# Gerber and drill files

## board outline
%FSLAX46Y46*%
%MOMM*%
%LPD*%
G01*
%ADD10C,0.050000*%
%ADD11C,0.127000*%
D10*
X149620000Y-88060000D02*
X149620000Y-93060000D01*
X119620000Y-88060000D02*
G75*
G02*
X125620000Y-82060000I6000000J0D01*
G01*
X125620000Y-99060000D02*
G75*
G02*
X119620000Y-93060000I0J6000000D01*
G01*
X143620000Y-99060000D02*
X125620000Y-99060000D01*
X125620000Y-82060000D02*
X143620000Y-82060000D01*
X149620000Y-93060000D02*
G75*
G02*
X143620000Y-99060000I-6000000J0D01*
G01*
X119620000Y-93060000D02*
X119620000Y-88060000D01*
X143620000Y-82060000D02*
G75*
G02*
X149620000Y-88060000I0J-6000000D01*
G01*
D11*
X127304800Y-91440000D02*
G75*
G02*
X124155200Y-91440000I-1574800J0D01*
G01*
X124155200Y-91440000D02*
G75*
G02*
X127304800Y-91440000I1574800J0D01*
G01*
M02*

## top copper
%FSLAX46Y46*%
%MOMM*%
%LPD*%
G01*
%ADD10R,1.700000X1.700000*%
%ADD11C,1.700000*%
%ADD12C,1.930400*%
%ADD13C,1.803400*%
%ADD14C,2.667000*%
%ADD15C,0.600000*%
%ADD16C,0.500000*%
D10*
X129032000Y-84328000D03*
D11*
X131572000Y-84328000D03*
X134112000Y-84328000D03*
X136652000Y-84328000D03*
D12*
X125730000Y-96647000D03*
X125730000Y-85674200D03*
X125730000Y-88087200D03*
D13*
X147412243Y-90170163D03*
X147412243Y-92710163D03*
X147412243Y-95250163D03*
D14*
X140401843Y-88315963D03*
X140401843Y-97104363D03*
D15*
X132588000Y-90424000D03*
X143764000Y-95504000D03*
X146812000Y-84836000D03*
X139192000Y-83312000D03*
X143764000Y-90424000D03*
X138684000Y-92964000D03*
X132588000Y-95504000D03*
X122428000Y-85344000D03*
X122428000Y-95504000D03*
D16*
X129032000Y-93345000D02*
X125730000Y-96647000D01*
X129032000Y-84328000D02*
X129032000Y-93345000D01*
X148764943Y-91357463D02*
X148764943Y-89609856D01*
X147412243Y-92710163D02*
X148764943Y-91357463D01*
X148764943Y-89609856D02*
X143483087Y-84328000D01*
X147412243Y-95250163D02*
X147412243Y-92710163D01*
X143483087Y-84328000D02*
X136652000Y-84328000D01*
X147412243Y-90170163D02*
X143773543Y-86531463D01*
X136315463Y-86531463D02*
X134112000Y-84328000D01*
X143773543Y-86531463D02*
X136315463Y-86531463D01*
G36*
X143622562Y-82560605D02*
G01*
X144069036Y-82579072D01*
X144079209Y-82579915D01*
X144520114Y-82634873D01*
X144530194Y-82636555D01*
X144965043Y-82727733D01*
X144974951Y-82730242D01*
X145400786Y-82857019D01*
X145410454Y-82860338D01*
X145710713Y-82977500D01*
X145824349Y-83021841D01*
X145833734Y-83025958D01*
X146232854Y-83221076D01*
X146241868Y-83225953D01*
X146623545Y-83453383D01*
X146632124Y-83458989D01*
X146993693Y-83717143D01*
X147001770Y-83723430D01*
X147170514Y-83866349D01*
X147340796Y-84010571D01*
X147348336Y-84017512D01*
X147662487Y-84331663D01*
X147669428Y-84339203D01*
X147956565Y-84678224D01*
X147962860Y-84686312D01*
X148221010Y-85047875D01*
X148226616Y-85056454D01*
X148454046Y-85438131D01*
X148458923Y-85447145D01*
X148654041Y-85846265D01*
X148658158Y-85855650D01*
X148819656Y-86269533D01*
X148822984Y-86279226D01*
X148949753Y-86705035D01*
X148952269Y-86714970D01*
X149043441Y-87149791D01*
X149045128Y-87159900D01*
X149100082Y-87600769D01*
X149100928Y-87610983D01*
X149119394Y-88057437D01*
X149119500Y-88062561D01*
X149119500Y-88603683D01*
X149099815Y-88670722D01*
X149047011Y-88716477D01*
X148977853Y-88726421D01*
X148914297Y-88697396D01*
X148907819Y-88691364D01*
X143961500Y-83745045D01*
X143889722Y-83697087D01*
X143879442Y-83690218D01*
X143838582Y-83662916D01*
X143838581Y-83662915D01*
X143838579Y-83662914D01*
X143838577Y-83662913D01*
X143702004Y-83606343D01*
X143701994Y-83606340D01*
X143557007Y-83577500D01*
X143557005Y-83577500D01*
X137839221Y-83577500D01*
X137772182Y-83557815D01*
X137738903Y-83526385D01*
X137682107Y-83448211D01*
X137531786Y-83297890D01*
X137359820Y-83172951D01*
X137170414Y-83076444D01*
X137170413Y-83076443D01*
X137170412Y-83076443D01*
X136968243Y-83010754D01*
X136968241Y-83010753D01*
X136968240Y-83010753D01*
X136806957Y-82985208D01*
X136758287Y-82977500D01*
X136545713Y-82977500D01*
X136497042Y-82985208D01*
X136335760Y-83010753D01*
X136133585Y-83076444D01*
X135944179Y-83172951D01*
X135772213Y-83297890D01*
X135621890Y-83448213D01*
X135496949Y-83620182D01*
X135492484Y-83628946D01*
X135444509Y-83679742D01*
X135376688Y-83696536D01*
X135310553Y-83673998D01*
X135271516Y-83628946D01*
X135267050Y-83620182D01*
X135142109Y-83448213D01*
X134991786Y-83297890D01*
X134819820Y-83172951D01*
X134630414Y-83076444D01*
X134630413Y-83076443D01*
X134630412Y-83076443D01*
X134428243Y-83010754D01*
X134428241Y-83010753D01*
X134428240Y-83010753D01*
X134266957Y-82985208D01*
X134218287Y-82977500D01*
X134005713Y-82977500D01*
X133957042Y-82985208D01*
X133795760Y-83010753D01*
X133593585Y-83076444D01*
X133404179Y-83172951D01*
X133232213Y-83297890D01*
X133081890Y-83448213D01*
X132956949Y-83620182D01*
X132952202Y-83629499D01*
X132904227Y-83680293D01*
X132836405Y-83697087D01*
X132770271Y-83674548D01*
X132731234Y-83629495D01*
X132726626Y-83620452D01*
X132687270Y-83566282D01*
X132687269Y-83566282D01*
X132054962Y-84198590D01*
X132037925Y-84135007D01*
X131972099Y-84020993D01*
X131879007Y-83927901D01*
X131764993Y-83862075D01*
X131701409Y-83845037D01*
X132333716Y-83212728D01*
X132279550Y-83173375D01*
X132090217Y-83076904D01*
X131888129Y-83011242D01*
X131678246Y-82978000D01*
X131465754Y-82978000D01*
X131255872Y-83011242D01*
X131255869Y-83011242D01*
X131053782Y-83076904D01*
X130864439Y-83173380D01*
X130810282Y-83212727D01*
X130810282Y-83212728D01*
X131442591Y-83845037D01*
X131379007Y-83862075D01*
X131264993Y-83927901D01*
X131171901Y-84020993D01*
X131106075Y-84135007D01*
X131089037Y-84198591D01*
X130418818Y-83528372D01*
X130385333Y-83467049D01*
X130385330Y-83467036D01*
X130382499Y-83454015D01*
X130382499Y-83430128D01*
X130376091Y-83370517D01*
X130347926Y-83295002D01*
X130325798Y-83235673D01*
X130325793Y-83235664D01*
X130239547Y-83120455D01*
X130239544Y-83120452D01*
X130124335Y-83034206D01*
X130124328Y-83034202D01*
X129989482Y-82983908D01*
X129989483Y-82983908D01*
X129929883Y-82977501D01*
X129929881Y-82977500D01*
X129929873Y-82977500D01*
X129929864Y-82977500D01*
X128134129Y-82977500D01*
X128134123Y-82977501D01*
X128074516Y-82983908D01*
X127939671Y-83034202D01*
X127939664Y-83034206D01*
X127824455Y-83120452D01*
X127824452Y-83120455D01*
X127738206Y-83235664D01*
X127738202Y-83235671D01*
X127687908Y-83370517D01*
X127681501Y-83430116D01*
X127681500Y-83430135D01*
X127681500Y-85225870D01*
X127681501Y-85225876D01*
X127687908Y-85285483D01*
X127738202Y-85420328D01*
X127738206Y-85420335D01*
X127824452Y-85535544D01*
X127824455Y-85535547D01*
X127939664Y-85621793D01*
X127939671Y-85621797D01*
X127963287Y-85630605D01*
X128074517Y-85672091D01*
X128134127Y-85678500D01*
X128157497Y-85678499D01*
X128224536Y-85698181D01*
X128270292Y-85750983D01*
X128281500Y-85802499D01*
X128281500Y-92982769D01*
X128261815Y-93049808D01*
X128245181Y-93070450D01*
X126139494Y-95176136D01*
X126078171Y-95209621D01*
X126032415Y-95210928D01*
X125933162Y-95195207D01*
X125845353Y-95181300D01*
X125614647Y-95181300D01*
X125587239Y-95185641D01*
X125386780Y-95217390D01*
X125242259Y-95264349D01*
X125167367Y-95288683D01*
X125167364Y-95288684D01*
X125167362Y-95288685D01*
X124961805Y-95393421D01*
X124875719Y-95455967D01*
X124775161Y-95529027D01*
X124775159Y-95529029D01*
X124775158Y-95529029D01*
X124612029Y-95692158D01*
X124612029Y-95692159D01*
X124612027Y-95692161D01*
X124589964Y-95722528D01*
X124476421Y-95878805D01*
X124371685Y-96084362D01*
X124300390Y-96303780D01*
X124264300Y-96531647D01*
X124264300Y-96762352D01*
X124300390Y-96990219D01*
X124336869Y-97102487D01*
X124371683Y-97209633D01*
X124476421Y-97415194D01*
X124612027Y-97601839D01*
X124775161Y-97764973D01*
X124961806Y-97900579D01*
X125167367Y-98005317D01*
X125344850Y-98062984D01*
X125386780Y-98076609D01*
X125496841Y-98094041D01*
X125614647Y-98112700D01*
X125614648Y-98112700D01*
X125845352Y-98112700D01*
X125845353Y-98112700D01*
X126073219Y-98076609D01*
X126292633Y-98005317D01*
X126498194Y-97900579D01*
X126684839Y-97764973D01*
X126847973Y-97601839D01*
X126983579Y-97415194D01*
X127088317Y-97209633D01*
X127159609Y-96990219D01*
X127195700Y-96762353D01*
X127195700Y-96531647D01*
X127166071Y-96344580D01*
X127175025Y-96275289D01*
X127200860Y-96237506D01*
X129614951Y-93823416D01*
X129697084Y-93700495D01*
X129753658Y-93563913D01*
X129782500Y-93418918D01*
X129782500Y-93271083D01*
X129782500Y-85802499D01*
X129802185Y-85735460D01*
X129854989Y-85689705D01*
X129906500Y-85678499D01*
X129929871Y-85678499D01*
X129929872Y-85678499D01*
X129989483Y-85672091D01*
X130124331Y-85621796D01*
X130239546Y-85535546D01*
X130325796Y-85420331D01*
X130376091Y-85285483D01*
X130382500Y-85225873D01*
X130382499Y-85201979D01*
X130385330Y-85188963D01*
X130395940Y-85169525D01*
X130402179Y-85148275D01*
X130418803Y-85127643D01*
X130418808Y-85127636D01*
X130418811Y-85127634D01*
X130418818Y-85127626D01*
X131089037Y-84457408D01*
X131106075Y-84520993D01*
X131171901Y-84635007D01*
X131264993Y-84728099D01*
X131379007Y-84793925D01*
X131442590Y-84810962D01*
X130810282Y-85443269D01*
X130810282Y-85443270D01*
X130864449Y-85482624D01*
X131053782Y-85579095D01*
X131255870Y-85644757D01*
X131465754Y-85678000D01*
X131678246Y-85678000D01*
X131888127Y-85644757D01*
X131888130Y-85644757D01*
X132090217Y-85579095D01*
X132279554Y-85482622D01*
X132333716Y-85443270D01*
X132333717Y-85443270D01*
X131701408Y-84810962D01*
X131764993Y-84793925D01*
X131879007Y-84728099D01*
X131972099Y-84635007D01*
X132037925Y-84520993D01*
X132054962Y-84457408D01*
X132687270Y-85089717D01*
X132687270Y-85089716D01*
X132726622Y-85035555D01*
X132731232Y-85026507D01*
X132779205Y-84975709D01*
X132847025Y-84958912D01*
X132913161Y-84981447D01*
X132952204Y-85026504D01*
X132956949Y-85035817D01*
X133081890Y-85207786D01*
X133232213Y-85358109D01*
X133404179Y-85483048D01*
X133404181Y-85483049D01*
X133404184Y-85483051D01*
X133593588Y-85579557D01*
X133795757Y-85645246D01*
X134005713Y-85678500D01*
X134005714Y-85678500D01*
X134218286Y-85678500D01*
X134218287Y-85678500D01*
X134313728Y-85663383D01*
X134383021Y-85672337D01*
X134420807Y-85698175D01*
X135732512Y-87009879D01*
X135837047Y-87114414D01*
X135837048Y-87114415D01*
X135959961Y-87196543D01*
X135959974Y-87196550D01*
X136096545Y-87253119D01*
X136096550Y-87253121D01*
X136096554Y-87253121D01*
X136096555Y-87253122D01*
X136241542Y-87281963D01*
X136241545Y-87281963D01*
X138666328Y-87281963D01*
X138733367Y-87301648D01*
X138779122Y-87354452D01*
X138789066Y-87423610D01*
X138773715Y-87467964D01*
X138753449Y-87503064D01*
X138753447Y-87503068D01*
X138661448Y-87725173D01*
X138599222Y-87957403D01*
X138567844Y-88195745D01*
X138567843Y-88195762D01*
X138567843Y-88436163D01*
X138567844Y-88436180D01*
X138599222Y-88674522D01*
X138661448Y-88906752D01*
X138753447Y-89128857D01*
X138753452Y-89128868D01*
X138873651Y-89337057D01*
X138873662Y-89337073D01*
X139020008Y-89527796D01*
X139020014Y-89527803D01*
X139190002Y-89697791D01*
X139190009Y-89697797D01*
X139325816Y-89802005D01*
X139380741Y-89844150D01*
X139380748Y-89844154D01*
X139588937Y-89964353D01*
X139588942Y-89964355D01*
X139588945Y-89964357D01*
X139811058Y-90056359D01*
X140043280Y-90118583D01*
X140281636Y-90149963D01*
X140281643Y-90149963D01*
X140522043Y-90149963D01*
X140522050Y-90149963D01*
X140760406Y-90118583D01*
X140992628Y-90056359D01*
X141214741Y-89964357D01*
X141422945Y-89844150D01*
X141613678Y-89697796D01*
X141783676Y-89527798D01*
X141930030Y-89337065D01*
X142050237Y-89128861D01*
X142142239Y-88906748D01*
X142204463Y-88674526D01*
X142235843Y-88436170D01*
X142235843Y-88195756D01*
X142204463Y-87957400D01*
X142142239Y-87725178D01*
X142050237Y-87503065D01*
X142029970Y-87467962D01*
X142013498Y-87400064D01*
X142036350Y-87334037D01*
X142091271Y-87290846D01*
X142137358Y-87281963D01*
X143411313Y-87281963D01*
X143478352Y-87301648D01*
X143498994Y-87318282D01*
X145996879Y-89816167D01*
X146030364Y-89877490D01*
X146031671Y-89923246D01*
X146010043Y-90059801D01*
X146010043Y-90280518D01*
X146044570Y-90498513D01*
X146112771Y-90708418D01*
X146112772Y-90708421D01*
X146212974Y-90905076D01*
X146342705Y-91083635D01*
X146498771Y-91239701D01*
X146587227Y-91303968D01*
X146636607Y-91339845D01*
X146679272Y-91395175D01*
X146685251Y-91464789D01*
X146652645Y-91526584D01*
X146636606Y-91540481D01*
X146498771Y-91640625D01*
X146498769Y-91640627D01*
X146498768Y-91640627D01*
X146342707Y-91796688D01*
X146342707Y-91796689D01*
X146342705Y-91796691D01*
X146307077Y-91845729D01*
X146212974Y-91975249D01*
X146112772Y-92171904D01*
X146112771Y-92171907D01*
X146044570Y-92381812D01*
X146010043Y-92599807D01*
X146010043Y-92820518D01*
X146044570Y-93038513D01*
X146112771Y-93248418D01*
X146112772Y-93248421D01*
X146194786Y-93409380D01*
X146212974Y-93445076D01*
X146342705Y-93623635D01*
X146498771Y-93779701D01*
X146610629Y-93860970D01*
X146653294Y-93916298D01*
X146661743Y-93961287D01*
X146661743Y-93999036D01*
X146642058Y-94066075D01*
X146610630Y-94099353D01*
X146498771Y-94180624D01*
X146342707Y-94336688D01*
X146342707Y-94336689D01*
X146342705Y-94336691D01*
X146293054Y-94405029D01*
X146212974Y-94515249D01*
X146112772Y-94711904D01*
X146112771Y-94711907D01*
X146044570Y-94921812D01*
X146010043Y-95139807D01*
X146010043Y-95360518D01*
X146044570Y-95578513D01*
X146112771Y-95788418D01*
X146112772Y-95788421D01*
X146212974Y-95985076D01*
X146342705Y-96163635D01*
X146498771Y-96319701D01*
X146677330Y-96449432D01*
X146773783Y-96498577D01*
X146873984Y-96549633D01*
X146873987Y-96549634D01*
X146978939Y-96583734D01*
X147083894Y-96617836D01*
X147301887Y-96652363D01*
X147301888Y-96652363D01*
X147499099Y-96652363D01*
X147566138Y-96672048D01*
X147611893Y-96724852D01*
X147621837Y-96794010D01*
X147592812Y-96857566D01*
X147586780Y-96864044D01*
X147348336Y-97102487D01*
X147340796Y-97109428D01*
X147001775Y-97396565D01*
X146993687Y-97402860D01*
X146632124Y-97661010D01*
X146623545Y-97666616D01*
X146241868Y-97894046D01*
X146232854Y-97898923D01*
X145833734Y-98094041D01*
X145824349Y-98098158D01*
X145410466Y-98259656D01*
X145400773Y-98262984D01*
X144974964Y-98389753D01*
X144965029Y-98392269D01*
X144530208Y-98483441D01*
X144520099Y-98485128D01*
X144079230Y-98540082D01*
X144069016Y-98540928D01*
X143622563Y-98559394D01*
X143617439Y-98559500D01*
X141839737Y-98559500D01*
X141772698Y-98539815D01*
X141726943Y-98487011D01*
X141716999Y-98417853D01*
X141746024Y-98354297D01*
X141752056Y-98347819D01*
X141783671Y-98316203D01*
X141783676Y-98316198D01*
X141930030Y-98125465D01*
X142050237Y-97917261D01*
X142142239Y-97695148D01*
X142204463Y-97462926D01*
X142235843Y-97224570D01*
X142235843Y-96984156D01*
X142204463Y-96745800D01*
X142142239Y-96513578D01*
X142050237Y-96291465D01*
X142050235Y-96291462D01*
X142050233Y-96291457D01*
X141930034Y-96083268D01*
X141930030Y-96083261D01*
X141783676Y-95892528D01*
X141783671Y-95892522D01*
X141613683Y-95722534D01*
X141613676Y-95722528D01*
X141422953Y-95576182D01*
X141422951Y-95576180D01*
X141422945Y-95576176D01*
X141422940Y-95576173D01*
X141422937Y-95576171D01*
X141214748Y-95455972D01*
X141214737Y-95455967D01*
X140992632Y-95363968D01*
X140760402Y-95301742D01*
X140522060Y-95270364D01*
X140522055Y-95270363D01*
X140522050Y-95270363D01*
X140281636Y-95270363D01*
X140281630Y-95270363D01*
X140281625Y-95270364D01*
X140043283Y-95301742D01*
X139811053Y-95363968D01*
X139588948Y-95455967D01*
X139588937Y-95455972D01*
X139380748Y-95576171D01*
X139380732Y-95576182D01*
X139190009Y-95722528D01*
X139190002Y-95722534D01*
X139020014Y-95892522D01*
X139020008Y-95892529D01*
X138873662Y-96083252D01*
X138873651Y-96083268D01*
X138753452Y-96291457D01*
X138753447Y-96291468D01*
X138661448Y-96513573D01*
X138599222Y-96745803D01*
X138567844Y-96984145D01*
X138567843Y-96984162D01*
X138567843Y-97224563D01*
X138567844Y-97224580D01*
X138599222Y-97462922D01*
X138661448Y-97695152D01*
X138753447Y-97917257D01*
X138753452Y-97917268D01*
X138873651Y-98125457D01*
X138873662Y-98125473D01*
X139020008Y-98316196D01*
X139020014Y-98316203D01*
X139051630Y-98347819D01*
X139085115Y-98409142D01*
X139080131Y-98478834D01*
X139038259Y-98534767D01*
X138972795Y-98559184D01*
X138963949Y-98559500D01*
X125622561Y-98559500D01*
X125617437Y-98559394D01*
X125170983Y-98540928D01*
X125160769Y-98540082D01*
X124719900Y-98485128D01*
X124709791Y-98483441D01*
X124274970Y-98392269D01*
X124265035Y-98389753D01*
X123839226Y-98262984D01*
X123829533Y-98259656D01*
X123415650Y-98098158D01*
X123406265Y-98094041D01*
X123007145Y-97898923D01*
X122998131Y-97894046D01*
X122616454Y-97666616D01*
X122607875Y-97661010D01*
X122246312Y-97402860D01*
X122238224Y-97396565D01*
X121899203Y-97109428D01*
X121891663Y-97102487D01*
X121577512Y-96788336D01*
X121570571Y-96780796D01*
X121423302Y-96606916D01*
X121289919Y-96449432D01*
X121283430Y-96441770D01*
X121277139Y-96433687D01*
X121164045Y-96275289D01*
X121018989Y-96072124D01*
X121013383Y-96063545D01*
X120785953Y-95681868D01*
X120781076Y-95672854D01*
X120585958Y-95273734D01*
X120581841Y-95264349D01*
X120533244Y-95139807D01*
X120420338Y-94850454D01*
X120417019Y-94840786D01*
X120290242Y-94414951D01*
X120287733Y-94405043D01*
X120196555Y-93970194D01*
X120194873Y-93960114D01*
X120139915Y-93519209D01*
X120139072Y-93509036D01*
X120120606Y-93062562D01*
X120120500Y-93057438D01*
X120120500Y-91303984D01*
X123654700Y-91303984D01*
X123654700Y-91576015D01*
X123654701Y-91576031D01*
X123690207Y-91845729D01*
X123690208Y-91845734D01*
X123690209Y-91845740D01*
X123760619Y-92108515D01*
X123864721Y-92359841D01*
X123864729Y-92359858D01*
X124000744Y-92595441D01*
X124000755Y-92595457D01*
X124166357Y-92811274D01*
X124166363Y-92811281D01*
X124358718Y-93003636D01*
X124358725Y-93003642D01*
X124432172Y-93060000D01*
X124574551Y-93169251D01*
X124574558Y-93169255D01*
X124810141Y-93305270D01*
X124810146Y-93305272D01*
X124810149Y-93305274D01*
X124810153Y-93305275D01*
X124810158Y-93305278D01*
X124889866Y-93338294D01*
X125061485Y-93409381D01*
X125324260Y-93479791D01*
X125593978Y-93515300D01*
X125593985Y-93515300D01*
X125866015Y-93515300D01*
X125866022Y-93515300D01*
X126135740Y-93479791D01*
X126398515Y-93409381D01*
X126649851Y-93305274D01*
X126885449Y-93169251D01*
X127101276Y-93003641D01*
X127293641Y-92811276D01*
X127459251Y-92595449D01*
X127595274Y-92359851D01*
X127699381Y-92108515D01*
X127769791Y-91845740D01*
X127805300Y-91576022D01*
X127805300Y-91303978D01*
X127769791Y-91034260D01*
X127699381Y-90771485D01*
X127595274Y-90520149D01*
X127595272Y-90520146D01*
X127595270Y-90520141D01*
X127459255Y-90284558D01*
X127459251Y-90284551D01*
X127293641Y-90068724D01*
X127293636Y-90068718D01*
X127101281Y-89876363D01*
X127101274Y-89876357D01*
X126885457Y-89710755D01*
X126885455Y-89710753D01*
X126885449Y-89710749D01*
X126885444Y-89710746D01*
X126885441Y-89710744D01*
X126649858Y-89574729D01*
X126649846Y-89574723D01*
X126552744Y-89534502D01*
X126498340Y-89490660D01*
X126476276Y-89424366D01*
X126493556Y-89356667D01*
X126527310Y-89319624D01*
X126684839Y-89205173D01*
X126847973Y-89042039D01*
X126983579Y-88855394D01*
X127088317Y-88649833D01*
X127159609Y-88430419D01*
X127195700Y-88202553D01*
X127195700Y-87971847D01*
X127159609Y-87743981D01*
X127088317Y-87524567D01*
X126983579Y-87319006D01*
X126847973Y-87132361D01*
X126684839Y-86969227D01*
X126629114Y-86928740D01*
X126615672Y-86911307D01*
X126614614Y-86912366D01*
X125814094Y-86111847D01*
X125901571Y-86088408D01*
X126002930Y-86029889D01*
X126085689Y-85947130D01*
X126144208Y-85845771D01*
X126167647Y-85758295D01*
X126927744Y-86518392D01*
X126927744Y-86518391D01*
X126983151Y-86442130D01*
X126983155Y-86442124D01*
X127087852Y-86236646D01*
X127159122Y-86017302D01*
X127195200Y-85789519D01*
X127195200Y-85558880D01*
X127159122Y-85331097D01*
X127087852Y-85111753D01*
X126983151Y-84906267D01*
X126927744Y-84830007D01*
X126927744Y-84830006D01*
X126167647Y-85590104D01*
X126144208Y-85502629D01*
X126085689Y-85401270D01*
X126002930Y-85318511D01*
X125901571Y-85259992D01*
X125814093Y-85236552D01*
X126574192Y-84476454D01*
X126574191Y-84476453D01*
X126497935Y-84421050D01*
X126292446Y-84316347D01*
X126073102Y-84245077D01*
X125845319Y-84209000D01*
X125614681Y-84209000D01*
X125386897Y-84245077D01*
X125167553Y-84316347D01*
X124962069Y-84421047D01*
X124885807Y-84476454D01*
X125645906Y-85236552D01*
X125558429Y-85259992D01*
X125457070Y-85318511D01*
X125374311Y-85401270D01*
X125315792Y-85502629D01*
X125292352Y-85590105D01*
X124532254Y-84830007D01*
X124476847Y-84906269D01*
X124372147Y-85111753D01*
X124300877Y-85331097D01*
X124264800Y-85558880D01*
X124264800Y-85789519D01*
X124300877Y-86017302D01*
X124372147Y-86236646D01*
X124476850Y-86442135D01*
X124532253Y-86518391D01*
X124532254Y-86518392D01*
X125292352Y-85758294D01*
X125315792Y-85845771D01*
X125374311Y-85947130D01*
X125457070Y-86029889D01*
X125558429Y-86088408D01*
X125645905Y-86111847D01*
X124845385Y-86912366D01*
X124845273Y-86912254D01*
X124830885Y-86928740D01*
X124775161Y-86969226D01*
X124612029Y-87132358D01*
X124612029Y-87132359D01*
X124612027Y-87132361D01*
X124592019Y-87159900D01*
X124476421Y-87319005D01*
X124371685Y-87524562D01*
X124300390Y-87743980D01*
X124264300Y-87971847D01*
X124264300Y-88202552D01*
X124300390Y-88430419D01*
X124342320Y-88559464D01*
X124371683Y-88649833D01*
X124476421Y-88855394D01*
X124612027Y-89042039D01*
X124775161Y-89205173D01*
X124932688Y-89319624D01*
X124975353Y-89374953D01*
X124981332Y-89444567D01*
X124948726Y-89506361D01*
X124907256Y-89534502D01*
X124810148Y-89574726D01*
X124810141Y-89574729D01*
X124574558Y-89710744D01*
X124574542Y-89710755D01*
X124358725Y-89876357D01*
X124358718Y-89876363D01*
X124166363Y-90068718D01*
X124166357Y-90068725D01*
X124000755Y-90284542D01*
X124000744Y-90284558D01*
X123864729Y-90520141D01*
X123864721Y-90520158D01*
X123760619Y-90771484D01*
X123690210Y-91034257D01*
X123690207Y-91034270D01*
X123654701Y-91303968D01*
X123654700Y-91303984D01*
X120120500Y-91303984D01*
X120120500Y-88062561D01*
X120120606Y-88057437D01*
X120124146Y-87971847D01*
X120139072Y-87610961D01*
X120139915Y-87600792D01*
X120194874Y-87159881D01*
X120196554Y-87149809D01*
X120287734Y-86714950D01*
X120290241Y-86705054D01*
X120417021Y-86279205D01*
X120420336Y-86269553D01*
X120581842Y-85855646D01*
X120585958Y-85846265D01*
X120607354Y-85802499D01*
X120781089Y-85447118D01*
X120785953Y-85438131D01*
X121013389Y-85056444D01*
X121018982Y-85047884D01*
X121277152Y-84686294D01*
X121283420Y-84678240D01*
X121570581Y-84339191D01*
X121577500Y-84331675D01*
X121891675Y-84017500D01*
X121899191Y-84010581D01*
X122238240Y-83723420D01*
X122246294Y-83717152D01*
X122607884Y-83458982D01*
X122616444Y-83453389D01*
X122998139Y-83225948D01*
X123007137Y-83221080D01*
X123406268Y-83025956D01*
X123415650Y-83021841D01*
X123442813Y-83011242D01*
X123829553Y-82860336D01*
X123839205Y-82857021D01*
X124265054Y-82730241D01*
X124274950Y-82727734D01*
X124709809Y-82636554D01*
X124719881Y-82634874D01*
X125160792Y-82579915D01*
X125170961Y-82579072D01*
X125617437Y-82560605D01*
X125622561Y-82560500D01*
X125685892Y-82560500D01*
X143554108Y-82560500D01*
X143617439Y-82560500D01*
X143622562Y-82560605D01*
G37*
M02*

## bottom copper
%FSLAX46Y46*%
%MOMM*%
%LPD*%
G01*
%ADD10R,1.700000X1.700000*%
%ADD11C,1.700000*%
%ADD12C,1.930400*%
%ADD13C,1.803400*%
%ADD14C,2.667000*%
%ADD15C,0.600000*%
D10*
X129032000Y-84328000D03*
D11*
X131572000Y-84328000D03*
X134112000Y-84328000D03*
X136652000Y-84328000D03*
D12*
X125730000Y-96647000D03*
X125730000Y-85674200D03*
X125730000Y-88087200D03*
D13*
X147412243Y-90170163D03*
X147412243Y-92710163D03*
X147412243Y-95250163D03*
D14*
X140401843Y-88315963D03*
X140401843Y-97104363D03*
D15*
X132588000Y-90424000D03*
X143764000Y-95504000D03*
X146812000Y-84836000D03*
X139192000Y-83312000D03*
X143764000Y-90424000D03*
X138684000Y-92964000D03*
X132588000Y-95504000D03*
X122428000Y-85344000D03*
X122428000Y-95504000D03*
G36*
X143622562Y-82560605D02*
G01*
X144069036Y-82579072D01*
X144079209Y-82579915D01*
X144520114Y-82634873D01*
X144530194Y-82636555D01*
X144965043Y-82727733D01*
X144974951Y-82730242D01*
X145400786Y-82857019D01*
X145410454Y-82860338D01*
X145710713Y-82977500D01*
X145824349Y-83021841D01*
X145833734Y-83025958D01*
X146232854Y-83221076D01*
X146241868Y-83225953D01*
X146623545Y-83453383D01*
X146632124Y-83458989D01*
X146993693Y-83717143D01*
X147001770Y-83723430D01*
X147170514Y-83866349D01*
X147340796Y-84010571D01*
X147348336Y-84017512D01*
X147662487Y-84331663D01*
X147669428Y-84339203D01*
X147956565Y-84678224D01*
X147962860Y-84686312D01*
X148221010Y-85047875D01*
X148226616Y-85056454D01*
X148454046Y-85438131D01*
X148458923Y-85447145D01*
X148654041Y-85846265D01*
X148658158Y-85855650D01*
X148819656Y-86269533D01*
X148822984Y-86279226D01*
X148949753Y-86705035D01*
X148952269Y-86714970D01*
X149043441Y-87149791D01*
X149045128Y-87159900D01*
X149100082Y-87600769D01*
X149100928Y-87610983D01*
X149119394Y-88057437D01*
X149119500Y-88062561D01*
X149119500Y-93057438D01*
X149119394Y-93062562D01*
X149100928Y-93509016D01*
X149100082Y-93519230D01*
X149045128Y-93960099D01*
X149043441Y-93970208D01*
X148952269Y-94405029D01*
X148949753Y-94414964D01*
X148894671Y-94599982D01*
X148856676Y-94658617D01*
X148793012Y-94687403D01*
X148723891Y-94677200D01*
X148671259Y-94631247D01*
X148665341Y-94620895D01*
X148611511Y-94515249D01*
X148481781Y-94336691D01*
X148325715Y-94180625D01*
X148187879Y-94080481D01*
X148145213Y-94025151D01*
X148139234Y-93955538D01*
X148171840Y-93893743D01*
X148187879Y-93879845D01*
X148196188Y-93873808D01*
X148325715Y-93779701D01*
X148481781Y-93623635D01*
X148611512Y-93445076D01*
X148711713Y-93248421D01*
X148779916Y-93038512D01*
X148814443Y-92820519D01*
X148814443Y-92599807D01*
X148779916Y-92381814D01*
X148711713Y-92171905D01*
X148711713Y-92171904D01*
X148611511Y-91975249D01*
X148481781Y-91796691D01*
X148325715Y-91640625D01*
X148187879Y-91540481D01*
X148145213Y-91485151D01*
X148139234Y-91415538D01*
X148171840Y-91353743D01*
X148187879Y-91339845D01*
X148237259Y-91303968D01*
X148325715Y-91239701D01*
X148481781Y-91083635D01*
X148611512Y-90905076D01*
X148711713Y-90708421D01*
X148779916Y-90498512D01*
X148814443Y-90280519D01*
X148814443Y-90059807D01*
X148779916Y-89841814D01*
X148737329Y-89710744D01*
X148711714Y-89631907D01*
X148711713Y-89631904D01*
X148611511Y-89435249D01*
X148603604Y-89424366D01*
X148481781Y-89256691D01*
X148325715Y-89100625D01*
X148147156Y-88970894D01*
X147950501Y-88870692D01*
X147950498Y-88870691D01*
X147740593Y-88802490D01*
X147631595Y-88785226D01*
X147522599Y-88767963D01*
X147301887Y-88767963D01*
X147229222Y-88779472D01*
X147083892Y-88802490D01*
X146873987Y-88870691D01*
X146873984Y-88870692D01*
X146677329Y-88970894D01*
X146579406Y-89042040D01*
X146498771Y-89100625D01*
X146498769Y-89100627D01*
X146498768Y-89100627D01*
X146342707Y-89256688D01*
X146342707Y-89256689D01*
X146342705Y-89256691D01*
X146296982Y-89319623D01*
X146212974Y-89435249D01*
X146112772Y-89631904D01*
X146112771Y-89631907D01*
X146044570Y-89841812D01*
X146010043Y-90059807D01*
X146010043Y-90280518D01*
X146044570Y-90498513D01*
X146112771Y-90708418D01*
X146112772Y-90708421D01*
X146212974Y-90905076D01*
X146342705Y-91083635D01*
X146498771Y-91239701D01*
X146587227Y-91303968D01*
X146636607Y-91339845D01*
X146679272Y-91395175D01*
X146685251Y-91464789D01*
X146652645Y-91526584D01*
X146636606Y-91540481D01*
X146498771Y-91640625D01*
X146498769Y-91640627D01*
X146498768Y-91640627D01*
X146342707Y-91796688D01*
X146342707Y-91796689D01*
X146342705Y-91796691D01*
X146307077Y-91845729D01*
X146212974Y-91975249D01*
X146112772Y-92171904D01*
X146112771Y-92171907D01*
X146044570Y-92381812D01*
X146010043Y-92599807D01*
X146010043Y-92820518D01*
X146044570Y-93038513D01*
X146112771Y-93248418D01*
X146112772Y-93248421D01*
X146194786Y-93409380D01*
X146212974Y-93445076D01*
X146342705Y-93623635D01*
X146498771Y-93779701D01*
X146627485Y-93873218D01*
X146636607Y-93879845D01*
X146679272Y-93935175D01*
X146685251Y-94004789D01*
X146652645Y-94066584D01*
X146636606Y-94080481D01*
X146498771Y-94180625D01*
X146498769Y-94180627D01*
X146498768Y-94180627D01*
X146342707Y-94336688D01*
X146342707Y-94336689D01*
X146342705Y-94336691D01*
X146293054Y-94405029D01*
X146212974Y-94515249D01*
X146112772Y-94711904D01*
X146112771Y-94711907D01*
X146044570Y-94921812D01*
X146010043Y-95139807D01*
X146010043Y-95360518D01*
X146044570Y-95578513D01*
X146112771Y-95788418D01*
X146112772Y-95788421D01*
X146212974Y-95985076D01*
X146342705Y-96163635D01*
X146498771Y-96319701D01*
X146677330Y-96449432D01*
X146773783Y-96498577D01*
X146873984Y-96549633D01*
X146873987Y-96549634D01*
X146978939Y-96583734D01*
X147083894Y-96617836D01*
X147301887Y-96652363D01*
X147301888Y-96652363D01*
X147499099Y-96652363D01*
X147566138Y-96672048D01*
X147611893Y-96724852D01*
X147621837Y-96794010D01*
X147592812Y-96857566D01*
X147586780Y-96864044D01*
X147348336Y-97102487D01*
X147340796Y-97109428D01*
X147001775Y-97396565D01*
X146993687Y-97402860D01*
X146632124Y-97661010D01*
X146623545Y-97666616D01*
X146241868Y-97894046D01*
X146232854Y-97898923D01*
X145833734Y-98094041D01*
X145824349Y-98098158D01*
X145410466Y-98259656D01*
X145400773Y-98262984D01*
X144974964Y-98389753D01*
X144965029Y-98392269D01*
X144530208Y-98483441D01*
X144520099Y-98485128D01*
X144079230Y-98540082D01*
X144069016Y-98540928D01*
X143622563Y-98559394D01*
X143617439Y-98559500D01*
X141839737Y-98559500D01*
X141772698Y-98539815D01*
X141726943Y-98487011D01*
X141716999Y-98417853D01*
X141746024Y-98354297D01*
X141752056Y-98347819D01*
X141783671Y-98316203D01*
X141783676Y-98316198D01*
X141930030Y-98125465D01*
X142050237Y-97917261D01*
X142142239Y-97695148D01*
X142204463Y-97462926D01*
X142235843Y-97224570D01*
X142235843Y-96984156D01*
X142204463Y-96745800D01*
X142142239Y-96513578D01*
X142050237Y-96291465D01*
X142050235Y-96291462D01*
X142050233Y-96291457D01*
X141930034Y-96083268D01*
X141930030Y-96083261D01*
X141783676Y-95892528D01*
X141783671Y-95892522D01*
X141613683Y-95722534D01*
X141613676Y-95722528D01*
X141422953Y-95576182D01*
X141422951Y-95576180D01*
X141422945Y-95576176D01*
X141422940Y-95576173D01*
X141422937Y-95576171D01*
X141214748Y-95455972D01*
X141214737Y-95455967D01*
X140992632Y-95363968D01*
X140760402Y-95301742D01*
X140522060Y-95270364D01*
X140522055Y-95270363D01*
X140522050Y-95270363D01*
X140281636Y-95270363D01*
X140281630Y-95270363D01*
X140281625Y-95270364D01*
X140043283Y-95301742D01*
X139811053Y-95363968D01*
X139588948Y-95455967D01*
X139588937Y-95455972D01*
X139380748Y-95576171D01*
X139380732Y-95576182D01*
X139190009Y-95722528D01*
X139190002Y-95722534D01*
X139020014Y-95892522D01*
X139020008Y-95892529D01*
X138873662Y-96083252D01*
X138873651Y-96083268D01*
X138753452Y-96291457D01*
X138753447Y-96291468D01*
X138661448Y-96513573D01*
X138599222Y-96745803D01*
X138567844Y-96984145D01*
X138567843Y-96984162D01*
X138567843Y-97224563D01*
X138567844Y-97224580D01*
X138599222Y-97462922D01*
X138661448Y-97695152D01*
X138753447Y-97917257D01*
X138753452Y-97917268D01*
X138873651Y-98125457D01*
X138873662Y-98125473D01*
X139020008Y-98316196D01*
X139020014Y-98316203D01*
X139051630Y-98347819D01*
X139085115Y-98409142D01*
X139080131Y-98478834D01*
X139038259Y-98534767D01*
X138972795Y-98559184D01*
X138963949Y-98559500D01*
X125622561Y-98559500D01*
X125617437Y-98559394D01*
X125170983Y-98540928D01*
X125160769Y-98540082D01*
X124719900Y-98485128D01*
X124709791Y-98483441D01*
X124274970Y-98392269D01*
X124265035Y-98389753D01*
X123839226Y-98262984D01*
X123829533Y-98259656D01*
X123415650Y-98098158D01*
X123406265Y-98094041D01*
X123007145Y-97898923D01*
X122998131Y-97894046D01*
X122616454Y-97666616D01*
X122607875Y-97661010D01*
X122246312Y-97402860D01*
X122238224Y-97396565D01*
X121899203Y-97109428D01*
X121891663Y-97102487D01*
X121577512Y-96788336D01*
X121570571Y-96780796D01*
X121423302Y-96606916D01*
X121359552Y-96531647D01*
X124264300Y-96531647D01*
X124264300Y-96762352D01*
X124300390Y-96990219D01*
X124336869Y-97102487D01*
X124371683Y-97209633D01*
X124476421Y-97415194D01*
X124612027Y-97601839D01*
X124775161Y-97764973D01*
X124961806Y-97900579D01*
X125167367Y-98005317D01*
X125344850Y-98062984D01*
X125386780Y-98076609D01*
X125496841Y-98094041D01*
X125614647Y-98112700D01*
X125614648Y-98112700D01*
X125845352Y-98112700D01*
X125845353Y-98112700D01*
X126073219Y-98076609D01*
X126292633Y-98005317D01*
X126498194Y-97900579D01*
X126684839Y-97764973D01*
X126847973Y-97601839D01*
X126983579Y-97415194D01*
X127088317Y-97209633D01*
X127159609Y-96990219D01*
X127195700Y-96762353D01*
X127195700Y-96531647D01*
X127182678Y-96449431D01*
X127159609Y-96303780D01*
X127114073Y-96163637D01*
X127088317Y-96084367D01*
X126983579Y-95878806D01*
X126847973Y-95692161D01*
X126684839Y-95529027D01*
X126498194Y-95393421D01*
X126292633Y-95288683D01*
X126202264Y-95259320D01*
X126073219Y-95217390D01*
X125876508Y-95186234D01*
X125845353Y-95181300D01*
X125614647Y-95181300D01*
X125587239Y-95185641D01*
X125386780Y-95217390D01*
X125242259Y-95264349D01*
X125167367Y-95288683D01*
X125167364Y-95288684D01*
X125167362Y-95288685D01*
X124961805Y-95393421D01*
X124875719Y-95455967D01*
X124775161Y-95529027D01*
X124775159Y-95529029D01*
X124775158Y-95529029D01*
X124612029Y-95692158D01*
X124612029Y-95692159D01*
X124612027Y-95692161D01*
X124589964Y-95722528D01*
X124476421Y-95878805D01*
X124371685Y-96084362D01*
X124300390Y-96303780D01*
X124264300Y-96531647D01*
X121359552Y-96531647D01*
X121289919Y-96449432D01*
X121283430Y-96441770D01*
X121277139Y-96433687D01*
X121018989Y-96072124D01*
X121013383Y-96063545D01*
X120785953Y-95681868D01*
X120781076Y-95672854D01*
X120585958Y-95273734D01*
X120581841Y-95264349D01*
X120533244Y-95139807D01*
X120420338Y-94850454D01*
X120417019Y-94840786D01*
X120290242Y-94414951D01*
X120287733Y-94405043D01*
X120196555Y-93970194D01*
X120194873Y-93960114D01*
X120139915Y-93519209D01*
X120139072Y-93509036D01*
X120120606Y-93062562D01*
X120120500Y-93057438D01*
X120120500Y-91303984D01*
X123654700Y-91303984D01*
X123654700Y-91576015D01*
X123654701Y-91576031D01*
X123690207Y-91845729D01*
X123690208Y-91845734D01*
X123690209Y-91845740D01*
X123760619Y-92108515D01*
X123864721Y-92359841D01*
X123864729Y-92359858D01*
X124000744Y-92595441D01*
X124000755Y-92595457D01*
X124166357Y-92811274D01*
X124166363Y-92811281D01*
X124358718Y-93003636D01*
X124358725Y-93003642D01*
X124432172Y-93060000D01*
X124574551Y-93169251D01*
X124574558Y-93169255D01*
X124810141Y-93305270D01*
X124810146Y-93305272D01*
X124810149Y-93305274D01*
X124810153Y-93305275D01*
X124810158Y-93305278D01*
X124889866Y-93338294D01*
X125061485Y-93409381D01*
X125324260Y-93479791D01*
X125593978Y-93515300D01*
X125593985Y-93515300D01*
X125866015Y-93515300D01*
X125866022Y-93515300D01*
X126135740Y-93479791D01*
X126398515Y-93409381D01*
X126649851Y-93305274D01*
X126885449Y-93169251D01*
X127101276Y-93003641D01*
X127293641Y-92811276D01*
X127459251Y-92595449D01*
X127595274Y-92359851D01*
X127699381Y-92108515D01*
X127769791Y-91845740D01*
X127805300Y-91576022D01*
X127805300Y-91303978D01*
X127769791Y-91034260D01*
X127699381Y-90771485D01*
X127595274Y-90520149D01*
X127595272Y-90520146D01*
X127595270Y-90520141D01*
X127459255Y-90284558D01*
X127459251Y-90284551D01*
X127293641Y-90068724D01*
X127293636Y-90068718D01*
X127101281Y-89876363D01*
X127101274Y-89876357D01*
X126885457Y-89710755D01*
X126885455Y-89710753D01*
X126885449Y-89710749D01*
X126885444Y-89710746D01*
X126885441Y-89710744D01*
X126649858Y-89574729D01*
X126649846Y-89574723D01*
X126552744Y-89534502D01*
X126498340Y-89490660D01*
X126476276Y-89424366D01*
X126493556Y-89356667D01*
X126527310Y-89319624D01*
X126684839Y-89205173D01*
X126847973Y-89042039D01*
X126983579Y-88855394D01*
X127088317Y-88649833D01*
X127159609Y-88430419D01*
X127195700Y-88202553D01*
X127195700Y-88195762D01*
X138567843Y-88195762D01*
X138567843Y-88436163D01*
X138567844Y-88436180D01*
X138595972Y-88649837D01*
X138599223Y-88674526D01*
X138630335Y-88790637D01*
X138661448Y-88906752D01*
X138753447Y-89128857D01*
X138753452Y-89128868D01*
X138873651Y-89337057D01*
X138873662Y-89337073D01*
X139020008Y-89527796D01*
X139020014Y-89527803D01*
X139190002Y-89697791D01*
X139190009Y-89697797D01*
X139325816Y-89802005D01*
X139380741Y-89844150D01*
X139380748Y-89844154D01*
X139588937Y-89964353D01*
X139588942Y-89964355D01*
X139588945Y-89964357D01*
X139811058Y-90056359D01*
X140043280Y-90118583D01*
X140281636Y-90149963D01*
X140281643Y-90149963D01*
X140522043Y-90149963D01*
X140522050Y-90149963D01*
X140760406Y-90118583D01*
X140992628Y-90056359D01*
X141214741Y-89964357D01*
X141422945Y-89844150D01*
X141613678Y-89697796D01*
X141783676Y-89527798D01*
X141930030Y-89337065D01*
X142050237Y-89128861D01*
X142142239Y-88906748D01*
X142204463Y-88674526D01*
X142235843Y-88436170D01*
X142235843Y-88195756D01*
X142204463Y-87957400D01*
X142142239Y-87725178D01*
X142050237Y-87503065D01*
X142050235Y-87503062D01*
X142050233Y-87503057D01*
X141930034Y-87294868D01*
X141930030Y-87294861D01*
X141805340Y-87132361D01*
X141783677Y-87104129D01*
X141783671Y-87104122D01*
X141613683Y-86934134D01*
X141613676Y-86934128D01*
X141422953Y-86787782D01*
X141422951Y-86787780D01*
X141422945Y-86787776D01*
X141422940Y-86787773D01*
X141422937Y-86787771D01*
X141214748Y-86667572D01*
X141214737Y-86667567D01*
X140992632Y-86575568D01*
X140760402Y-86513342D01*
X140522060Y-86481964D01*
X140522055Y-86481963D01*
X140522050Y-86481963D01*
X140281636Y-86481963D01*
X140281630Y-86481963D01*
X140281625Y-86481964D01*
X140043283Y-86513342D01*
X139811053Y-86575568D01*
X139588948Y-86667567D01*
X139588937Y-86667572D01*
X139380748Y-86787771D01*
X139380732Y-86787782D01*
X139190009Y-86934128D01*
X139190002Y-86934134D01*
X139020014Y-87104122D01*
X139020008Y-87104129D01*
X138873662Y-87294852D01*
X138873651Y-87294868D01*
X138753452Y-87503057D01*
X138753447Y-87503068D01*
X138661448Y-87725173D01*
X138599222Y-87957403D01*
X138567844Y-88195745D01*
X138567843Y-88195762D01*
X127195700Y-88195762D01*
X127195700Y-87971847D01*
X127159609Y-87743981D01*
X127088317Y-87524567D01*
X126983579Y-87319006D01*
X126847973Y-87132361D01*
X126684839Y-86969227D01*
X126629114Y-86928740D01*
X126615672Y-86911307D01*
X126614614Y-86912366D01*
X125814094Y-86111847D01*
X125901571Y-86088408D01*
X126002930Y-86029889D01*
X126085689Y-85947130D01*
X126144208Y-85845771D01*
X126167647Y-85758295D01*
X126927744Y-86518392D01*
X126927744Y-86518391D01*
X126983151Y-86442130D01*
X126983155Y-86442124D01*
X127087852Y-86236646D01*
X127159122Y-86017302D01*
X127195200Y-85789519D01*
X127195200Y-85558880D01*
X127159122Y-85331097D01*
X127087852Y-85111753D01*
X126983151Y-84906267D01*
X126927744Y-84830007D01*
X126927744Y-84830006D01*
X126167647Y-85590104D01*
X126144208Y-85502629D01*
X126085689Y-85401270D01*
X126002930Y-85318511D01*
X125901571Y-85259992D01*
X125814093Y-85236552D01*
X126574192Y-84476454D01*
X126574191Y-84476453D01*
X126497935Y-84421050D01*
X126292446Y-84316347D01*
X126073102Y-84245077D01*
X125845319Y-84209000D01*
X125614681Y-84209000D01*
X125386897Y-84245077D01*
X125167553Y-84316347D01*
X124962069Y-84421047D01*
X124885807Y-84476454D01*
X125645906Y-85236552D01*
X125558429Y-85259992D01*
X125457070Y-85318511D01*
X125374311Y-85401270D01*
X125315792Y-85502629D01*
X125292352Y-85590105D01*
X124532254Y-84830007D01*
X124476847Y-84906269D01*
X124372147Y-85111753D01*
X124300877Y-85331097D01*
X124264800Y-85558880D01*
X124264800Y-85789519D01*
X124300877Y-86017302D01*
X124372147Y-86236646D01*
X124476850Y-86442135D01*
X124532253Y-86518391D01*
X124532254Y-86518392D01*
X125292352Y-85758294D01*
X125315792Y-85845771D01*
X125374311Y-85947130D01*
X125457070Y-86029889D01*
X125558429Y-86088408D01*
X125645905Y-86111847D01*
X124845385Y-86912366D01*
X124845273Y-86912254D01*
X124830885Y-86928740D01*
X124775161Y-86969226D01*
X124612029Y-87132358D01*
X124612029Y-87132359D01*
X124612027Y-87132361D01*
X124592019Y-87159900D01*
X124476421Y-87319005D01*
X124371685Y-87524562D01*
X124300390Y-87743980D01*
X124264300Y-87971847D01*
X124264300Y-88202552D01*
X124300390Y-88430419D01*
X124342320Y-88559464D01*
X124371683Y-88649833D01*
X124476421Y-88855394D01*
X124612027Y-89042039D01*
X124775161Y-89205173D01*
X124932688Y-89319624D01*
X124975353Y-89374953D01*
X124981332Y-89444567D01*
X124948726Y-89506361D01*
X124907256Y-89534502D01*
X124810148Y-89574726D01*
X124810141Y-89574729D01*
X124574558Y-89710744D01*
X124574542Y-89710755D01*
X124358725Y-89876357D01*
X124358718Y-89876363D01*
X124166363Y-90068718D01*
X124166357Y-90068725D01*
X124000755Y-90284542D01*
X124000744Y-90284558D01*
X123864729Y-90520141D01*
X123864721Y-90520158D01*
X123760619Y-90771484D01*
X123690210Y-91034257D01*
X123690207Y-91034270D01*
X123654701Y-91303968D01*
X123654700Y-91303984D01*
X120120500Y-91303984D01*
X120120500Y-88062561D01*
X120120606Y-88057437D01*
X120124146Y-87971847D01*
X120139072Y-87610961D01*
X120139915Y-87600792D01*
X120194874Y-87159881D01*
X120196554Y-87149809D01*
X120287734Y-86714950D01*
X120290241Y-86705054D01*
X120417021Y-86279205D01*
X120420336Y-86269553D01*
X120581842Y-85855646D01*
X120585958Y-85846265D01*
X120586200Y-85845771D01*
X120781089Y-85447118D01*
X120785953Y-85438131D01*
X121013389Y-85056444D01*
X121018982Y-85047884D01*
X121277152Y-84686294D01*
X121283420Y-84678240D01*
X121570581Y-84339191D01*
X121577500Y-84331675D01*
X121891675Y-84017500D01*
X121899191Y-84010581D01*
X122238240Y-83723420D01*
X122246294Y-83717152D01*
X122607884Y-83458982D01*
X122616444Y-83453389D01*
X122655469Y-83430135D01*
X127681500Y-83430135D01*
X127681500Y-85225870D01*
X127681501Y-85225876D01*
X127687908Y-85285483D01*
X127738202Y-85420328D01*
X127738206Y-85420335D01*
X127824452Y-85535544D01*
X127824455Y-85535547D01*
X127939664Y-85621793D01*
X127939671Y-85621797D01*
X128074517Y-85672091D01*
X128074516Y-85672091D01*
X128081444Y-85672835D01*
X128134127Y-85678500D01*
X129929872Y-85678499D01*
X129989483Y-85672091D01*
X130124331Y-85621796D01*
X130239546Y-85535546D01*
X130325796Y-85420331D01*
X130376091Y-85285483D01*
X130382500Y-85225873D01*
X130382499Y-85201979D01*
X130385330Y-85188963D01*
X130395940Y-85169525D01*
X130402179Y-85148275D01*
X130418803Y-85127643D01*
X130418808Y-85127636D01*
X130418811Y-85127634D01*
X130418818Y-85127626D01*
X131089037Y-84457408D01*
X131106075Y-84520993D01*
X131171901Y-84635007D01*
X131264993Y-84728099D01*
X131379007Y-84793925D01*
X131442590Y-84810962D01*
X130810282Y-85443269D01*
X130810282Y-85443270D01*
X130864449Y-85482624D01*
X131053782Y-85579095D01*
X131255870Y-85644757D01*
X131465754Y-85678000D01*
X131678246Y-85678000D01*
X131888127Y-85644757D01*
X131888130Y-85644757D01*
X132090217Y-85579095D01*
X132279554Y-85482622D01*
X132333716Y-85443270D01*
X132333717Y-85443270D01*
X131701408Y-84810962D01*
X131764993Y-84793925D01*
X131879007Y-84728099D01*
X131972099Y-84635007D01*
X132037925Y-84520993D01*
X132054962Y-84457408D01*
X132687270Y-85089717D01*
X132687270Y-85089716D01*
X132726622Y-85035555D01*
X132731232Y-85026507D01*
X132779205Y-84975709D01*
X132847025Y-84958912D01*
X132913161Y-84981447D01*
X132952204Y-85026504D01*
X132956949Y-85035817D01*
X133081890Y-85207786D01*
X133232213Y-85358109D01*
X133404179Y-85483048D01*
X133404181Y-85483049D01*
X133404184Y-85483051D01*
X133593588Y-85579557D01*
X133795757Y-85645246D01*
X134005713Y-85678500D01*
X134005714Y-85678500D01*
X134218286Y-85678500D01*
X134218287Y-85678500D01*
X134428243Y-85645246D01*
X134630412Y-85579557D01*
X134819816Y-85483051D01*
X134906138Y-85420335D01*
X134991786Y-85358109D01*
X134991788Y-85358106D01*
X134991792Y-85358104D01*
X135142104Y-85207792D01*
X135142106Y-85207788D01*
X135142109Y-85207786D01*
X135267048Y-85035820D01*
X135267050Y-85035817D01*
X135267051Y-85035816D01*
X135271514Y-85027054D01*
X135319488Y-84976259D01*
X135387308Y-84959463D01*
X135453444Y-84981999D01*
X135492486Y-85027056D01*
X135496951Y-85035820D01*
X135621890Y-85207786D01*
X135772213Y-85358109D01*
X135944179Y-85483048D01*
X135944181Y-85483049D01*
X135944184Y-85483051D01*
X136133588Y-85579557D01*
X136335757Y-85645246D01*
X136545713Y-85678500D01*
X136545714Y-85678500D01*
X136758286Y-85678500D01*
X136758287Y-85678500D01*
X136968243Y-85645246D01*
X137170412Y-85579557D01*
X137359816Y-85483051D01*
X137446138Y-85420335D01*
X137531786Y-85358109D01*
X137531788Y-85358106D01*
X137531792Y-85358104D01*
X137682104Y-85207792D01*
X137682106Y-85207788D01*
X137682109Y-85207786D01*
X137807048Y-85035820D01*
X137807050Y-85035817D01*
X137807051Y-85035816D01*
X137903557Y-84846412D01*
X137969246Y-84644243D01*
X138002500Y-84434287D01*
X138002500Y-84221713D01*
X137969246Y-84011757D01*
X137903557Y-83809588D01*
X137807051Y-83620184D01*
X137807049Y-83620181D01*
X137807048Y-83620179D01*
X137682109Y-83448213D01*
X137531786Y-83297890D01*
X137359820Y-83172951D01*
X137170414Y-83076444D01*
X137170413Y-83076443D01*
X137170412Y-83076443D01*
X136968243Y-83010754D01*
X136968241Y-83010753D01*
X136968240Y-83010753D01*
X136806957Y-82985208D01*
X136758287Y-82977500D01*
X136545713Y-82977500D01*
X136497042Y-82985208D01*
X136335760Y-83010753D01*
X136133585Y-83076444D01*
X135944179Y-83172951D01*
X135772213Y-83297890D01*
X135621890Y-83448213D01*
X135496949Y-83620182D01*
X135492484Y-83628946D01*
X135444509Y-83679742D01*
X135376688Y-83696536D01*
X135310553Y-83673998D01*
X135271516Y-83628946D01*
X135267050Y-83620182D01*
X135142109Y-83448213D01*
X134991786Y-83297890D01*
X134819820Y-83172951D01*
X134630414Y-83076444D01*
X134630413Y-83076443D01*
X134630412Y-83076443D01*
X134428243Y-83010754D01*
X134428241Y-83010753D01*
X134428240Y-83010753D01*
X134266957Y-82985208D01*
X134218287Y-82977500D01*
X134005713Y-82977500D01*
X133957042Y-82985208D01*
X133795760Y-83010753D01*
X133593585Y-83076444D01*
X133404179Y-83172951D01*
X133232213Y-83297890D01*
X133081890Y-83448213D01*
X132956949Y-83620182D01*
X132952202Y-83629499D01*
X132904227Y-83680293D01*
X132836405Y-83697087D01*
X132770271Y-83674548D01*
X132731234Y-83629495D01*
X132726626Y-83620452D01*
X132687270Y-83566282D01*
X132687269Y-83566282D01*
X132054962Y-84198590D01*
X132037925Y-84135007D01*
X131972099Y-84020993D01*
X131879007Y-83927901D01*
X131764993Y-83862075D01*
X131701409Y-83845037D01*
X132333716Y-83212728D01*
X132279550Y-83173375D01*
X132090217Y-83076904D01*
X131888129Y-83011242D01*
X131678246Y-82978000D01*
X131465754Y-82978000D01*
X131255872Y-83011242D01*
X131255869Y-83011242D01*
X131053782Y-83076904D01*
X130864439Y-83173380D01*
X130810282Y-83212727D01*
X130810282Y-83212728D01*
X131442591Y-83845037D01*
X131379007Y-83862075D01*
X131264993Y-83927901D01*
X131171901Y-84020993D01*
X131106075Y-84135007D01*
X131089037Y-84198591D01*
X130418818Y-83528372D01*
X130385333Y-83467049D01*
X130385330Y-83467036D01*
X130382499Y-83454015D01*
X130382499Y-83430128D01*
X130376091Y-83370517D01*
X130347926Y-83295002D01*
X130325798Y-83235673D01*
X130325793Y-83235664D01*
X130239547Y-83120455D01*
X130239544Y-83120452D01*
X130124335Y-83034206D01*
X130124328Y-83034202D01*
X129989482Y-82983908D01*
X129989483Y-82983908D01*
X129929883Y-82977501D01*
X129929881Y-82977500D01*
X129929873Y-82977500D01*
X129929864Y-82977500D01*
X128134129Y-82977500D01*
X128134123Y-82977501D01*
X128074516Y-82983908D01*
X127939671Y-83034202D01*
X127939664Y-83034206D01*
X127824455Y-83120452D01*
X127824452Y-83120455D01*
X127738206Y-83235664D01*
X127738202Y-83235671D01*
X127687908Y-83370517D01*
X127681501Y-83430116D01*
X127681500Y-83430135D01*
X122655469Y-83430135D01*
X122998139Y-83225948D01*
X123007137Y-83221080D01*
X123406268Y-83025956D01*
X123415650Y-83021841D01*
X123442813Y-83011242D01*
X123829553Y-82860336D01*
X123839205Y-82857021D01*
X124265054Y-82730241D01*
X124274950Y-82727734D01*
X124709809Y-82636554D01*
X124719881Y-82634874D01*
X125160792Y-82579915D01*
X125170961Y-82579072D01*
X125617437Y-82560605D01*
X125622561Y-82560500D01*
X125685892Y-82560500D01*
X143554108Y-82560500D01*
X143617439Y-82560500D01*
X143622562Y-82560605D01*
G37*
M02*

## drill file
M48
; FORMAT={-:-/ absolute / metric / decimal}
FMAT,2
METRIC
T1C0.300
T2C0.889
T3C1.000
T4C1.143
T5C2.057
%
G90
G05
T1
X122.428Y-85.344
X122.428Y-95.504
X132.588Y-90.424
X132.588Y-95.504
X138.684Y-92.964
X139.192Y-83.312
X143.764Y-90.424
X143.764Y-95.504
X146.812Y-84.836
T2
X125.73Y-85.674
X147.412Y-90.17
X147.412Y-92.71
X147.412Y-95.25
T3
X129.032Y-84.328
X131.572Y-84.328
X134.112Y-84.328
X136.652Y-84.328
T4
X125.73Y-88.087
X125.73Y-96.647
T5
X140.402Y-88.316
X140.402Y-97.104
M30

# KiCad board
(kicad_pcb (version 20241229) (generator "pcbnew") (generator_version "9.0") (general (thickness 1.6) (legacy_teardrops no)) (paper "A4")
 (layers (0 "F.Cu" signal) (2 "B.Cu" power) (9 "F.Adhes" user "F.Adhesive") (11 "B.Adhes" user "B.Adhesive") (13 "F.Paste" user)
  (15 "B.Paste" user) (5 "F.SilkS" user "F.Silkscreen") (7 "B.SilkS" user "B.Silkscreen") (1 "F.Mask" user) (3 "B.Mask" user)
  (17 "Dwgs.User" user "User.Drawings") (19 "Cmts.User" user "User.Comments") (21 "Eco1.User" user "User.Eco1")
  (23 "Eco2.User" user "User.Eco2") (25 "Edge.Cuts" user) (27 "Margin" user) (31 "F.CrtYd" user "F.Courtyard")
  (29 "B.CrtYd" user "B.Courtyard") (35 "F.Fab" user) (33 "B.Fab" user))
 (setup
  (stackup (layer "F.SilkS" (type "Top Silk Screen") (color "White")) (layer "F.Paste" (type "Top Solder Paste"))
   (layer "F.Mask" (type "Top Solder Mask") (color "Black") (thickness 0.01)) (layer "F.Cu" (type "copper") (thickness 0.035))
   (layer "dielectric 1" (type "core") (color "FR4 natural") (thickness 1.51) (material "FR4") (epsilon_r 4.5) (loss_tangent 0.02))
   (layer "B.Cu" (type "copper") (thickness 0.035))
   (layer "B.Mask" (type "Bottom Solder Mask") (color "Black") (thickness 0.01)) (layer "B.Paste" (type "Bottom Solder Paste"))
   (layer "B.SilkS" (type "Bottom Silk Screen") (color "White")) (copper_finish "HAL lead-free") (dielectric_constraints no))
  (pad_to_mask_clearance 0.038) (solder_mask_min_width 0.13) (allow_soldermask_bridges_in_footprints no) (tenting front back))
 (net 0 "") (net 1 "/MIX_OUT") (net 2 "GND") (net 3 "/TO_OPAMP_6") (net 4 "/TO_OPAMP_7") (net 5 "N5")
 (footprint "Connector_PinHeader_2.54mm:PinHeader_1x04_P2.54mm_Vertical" (layer "F.Cu") (at 129.032 84.328 90)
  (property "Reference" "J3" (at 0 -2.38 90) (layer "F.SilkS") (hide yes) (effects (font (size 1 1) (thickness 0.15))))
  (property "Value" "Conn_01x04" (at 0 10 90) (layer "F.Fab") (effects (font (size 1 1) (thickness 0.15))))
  (pad "1" thru_hole rect (at 0 0 90) (size 1.7 1.7) (drill 1) (layers "*.Cu" "*.Mask") (remove_unused_layers no) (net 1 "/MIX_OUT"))
  (pad "2" thru_hole circle (at 0 2.54 90) (size 1.7 1.7) (drill 1) (layers "*.Cu" "*.Mask") (remove_unused_layers no) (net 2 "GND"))
  (pad "3" thru_hole circle (at 0 5.08 90) (size 1.7 1.7) (drill 1) (layers "*.Cu" "*.Mask") (remove_unused_layers no) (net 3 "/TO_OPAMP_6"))
  (pad "4" thru_hole circle (at 0 7.62 90) (size 1.7 1.7) (drill 1) (layers "*.Cu" "*.Mask") (remove_unused_layers no) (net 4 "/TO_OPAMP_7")))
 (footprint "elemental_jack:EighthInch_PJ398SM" (layer "B.Cu") (at 125.73 91.44 90)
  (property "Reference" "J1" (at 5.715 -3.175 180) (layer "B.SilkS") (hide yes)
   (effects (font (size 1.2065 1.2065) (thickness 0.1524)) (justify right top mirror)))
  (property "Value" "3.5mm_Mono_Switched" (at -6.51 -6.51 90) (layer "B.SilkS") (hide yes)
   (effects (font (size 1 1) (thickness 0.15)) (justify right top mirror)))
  (fp_circle (center 0 0) (end 1.5748 0) (stroke (width 0.127) (type solid)) (fill no) (layer "Edge.Cuts"))
  (pad "1" thru_hole circle (at -5.207 0 90) (size 1.9304 1.9304) (drill 1.143) (layers "*.Cu" "*.Mask") (remove_unused_layers no)
   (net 1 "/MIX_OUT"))
  (pad "2" thru_hole circle (at 5.7658 0 90) (size 1.9304 1.9304) (drill 0.889) (layers "*.Cu" "*.Mask") (remove_unused_layers no)
   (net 2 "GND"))
  (pad "3" thru_hole circle (at 3.3528 0 90) (size 1.9304 1.9304) (drill 1.143) (layers "*.Cu" "*.Mask") (remove_unused_layers no)
   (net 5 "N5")))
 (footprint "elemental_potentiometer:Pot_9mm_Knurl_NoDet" (layer "B.Cu") (at 140.4 92.71 90)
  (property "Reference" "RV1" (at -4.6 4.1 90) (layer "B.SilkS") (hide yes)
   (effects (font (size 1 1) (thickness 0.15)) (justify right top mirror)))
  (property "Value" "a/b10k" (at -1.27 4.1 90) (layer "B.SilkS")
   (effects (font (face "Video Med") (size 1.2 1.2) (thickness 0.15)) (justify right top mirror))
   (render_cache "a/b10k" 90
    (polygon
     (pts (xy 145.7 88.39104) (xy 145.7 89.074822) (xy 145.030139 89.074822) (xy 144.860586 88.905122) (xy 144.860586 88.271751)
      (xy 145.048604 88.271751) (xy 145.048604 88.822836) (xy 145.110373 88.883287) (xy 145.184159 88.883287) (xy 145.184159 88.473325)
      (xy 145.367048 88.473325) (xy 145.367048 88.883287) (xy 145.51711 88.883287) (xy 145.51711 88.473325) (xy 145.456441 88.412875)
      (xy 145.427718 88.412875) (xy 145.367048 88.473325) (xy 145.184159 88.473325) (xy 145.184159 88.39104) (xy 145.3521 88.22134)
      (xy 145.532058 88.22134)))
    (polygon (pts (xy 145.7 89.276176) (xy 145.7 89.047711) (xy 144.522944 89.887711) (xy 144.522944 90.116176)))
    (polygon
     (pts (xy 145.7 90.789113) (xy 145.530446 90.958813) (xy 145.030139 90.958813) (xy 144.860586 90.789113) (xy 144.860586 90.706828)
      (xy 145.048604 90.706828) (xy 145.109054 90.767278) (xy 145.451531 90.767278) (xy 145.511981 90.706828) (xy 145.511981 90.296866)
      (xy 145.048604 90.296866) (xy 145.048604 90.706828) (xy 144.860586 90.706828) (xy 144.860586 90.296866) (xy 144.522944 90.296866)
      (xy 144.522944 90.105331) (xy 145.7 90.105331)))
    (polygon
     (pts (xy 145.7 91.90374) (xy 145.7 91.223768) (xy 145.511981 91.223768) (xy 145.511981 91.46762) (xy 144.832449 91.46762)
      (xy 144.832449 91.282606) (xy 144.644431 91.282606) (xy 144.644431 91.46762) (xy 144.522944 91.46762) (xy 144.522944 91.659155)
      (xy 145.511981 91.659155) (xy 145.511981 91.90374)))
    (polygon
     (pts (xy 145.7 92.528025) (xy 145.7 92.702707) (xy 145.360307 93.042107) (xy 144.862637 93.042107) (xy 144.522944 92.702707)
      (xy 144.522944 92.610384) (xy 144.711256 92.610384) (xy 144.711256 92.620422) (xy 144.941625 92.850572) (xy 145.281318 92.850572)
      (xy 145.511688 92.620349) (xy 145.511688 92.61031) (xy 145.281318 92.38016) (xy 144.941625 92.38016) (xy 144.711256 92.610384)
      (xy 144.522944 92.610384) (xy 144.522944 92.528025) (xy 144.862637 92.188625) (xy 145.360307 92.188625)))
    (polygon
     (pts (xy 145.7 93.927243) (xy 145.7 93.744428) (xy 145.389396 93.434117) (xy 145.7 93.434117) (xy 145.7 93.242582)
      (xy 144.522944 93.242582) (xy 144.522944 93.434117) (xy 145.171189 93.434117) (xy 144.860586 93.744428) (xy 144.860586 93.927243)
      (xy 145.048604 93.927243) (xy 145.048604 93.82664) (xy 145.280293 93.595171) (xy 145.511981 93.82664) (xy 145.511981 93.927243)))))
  (pad "1" thru_hole circle (at 2.539837 7.012243 180) (size 1.8034 1.8034) (drill 0.889) (layers "*.Cu" "*.Mask") (remove_unused_layers no)
   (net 3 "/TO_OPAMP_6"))
  (pad "2" thru_hole circle (at -0.000163 7.012243 180) (size 1.8034 1.8034) (drill 0.889) (layers "*.Cu" "*.Mask")
   (remove_unused_layers no) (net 4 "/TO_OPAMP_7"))
  (pad "3" thru_hole circle (at -2.540163 7.012243 180) (size 1.8034 1.8034) (drill 0.889) (layers "*.Cu" "*.Mask")
   (remove_unused_layers no) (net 4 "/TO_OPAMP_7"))
  (pad "4" thru_hole circle (at 4.394037 0.001843 90) (size 2.667 2.667) (drill 2.0574) (layers "*.Cu" "*.Mask") (remove_unused_layers no))
  (pad "5" thru_hole circle (at -4.394363 0.001843 90) (size 2.667 2.667) (drill 2.0574) (layers "*.Cu" "*.Mask") (remove_unused_layers no)))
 (gr_line (start 149.62 88.06) (end 149.62 93.06) (stroke (width 0.05) (type default)) (layer "Edge.Cuts"))
 (gr_arc (start 119.62 88.06) (mid 121.377359 83.817359) (end 125.62 82.06) (stroke (width 0.05) (type default)) (layer "Edge.Cuts"))
 (gr_arc (start 125.62 99.06) (mid 121.377359 97.302641) (end 119.62 93.06) (stroke (width 0.05) (type default)) (layer "Edge.Cuts"))
 (gr_line (start 143.62 99.06) (end 125.62 99.06) (stroke (width 0.05) (type default)) (layer "Edge.Cuts"))
 (gr_line (start 125.62 82.06) (end 143.62 82.06) (stroke (width 0.05) (type default)) (layer "Edge.Cuts"))
 (gr_arc (start 149.62 93.06) (mid 147.862641 97.302641) (end 143.62 99.06) (stroke (width 0.05) (type default)) (layer "Edge.Cuts"))
 (gr_line (start 119.62 93.06) (end 119.62 88.06) (stroke (width 0.05) (type default)) (layer "Edge.Cuts"))
 (gr_arc (start 143.62 82.06) (mid 147.862641 83.817359) (end 149.62 88.06) (stroke (width 0.05) (type default)) (layer "Edge.Cuts"))
 (via (at 132.588 90.424) (size 0.6) (drill 0.3) (layers "F.Cu" "B.Cu") (free yes) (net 2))
 (via (at 143.764 95.504) (size 0.6) (drill 0.3) (layers "F.Cu" "B.Cu") (free yes) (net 2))
 (via (at 146.812 84.836) (size 0.6) (drill 0.3) (layers "F.Cu" "B.Cu") (free yes) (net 2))
 (via (at 139.192 83.312) (size 0.6) (drill 0.3) (layers "F.Cu" "B.Cu") (free yes) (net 2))
 (via (at 143.764 90.424) (size 0.6) (drill 0.3) (layers "F.Cu" "B.Cu") (free yes) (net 2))
 (via (at 138.684 92.964) (size 0.6) (drill 0.3) (layers "F.Cu" "B.Cu") (free yes) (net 2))
 (via (at 132.588 95.504) (size 0.6) (drill 0.3) (layers "F.Cu" "B.Cu") (free yes) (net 2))
 (via (at 122.428 85.344) (size 0.6) (drill 0.3) (layers "F.Cu" "B.Cu") (free yes) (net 2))
 (via (at 122.428 95.504) (size 0.6) (drill 0.3) (layers "F.Cu" "B.Cu") (free yes) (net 2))
 (segment (start 129.032 93.345) (end 125.73 96.647) (width 0.5) (layer "F.Cu") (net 1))
 (segment (start 129.032 84.328) (end 129.032 93.345) (width 0.5) (layer "F.Cu") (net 1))
 (segment (start 148.764943 91.357463) (end 148.764943 89.609856) (width 0.5) (layer "F.Cu") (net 4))
 (segment (start 147.412243 92.710163) (end 148.764943 91.357463) (width 0.5) (layer "F.Cu") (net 4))
 (segment (start 148.764943 89.609856) (end 143.483087 84.328) (width 0.5) (layer "F.Cu") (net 4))
 (segment (start 147.412243 95.250163) (end 147.412243 92.710163) (width 0.5) (layer "F.Cu") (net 4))
 (segment (start 143.483087 84.328) (end 136.652 84.328) (width 0.5) (layer "F.Cu") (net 4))
 (segment (start 147.412243 90.170163) (end 143.773543 86.531463) (width 0.5) (layer "F.Cu") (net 3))
 (segment (start 136.315463 86.531463) (end 134.112 84.328) (width 0.5) (layer "F.Cu") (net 3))
 (segment (start 143.773543 86.531463) (end 136.315463 86.531463) (width 0.5) (layer "F.Cu") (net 3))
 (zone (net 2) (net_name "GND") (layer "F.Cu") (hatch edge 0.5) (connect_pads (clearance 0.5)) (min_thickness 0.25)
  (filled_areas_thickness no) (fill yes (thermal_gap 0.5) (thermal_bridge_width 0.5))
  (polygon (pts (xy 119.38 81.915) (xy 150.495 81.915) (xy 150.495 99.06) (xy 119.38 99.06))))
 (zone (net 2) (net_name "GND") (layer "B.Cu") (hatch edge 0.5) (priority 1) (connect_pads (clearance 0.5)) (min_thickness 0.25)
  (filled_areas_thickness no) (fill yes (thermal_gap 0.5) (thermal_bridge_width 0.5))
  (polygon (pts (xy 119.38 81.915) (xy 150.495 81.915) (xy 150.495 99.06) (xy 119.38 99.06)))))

